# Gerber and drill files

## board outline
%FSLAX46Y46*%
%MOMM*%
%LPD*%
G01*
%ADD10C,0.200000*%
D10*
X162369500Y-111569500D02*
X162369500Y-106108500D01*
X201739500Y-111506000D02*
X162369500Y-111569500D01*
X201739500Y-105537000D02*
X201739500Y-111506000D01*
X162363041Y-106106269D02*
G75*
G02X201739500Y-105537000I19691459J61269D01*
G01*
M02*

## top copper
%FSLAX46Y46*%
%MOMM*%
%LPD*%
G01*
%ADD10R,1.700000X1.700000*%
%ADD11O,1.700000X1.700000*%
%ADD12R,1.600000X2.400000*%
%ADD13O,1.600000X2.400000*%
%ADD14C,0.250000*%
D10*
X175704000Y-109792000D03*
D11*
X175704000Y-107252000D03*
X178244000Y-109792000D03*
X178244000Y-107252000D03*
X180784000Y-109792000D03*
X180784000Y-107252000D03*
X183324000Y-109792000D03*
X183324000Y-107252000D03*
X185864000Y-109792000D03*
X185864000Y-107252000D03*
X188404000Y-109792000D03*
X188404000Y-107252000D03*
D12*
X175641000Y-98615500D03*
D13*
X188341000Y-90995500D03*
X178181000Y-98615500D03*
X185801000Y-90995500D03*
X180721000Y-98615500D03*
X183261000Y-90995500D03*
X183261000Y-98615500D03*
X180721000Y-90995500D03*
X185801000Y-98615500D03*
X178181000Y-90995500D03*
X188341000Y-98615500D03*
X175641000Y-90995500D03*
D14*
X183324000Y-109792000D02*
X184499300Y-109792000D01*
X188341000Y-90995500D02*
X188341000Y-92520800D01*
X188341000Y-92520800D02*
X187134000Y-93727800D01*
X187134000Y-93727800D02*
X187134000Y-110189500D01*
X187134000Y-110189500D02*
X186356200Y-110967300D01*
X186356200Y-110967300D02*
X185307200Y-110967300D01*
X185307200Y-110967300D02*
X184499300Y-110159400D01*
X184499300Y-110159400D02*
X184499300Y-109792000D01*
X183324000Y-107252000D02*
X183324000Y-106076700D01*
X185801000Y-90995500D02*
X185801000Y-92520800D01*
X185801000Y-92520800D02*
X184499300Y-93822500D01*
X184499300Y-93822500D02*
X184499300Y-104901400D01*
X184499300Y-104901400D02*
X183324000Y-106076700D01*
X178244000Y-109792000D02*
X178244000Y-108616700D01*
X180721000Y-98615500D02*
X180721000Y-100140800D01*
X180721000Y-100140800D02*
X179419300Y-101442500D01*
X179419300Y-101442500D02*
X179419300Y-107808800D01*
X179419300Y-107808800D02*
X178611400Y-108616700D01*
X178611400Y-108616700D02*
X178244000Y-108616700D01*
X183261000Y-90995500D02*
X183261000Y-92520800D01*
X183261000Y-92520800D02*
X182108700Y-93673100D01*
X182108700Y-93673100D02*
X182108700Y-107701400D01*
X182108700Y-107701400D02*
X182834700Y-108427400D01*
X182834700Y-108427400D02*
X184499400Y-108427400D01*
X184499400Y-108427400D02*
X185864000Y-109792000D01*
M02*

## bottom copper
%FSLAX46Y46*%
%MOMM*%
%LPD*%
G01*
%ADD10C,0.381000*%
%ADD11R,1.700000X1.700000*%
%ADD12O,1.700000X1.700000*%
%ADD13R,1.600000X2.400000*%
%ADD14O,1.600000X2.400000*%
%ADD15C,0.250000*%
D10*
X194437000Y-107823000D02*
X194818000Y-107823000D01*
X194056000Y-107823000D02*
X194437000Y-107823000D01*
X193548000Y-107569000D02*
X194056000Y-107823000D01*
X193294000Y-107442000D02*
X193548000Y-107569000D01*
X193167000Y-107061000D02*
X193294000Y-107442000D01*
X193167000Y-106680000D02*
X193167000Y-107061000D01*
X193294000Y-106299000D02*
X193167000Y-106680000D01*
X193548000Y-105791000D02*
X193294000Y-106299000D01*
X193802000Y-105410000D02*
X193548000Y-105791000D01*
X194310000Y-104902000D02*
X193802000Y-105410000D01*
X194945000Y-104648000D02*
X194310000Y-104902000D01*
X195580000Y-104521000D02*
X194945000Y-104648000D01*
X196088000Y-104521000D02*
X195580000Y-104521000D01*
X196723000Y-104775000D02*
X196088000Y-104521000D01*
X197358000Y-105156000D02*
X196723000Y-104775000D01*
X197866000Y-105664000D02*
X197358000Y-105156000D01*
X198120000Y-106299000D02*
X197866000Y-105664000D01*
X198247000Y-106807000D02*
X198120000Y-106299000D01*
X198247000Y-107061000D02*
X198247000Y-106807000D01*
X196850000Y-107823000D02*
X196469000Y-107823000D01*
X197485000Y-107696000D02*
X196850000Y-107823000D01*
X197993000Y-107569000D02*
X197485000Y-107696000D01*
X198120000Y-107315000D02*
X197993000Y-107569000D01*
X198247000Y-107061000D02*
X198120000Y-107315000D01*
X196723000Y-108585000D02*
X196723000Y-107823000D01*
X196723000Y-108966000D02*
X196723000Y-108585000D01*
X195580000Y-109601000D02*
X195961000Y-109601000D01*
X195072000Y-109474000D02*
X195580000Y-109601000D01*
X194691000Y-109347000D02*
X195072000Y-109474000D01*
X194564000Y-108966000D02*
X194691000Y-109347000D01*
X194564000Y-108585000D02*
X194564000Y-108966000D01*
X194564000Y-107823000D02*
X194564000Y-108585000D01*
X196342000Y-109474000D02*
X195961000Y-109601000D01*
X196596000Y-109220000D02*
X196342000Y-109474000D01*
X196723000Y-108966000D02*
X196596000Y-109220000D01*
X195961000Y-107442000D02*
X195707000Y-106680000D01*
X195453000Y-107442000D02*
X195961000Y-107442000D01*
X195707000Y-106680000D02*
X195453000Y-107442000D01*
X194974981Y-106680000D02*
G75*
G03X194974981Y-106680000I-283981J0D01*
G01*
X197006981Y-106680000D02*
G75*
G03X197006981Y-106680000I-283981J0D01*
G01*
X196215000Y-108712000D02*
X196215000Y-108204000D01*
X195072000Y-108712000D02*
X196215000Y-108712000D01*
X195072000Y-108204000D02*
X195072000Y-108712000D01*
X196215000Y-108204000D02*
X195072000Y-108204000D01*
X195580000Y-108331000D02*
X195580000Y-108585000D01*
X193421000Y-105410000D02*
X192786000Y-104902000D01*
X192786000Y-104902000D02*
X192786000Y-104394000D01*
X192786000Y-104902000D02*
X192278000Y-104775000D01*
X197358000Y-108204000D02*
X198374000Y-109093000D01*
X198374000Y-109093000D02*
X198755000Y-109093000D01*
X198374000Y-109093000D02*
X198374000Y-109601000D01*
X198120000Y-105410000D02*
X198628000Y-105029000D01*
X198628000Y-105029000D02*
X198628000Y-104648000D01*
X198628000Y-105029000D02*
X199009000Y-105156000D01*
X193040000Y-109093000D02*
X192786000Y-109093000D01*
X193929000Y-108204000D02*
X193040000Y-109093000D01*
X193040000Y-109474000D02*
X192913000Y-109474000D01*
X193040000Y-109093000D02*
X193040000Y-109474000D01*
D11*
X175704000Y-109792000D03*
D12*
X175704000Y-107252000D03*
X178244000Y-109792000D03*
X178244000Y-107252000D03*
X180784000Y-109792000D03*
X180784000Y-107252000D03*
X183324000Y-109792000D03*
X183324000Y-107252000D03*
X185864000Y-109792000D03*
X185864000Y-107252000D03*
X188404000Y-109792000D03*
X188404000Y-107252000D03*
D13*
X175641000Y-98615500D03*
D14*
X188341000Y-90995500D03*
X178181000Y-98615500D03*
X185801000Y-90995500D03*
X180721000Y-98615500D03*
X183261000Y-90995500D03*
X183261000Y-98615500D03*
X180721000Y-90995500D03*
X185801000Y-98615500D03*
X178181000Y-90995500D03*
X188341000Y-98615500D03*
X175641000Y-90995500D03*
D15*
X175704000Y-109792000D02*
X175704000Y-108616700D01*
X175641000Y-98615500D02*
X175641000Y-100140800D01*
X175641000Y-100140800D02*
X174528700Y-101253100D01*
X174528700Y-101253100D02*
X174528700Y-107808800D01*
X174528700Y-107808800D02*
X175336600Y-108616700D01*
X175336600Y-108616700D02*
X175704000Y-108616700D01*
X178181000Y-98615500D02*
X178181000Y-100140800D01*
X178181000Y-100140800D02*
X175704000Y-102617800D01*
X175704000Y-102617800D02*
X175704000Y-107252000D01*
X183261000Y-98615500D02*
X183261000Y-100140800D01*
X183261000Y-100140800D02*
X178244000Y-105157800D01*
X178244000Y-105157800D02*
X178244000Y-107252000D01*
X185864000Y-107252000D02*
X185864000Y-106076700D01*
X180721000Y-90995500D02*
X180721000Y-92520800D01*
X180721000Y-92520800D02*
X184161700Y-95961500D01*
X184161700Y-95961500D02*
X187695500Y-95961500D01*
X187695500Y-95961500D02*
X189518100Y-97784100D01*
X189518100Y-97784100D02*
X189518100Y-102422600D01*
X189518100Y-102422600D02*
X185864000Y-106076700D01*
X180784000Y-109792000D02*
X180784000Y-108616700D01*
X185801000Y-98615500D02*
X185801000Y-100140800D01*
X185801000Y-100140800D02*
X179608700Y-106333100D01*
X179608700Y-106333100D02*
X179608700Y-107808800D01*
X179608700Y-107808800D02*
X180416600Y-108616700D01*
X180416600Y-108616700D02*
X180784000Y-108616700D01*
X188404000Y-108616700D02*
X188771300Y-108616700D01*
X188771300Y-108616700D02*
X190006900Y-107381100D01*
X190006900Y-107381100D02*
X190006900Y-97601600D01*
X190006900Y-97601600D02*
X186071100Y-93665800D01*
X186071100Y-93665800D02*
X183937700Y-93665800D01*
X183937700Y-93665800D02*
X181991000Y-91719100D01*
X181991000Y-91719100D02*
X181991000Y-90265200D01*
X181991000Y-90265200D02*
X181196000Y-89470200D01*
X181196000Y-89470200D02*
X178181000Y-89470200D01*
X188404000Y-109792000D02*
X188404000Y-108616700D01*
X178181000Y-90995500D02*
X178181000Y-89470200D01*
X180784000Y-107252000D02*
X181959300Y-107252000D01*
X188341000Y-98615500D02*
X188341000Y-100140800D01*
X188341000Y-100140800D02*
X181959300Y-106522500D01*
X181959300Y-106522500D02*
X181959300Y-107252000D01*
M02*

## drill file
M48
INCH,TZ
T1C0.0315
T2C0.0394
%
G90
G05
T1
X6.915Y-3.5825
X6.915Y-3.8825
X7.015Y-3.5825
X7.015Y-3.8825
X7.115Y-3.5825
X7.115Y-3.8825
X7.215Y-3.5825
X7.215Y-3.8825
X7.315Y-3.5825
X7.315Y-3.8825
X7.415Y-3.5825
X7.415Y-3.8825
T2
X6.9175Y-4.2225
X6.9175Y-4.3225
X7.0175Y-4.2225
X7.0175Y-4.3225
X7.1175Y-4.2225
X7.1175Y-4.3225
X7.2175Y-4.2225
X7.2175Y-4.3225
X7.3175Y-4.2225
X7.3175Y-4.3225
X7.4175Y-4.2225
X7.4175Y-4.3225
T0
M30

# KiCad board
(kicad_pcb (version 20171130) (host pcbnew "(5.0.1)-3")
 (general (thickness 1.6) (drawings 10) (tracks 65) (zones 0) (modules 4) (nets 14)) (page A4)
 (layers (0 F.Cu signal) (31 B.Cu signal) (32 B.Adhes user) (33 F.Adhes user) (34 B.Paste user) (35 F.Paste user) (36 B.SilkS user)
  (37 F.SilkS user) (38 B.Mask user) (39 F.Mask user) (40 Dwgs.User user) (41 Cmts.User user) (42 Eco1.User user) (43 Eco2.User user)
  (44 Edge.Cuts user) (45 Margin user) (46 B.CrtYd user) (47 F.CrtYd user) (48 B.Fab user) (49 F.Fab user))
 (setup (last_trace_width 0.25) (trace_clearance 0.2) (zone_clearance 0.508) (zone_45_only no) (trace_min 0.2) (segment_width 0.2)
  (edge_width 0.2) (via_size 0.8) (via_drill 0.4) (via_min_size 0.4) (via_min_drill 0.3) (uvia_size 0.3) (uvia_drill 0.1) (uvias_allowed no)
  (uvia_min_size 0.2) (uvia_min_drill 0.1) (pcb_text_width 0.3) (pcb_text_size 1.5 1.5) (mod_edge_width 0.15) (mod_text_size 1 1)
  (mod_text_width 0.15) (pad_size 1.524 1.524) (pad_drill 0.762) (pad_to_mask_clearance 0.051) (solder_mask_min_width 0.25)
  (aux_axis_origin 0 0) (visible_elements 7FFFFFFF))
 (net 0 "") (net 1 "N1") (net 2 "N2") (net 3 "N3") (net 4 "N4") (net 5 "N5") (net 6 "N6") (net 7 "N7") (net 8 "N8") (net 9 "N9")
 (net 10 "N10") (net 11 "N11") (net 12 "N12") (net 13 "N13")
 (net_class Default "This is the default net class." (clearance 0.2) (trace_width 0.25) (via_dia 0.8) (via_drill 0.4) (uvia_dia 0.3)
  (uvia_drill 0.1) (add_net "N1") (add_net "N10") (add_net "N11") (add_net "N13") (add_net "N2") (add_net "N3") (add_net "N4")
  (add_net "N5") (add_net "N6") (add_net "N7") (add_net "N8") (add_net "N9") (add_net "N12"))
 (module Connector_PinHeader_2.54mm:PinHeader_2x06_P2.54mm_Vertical (layer F.Cu) (at 175.704 109.792 90)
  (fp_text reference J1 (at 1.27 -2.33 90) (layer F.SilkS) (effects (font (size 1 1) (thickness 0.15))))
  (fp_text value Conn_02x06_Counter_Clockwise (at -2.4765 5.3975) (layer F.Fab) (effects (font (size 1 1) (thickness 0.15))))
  (pad 1 thru_hole rect (at 0 0 90) (size 1.7 1.7) (drill 1) (layers *.Cu *.Mask) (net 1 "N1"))
  (pad 2 thru_hole oval (at 2.54 0 90) (size 1.7 1.7) (drill 1) (layers *.Cu *.Mask) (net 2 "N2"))
  (pad 3 thru_hole oval (at 0 2.54 90) (size 1.7 1.7) (drill 1) (layers *.Cu *.Mask) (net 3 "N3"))
  (pad 4 thru_hole oval (at 2.54 2.54 90) (size 1.7 1.7) (drill 1) (layers *.Cu *.Mask) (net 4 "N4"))
  (pad 5 thru_hole oval (at 0 5.08 90) (size 1.7 1.7) (drill 1) (layers *.Cu *.Mask) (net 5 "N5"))
  (pad 6 thru_hole oval (at 2.54 5.08 90) (size 1.7 1.7) (drill 1) (layers *.Cu *.Mask) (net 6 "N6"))
  (pad 7 thru_hole oval (at 0 7.62 90) (size 1.7 1.7) (drill 1) (layers *.Cu *.Mask) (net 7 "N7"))
  (pad 8 thru_hole oval (at 2.54 7.62 90) (size 1.7 1.7) (drill 1) (layers *.Cu *.Mask) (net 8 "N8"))
  (pad 9 thru_hole oval (at 0 10.16 90) (size 1.7 1.7) (drill 1) (layers *.Cu *.Mask) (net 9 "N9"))
  (pad 10 thru_hole oval (at 2.54 10.16 90) (size 1.7 1.7) (drill 1) (layers *.Cu *.Mask) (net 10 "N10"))
  (pad 11 thru_hole oval (at 0 12.7 90) (size 1.7 1.7) (drill 1) (layers *.Cu *.Mask) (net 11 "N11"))
  (pad 12 thru_hole oval (at 2.54 12.7 90) (size 1.7 1.7) (drill 1) (layers *.Cu *.Mask) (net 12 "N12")))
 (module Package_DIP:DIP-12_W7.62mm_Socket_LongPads (layer F.Cu) (at 175.641 98.6155 90)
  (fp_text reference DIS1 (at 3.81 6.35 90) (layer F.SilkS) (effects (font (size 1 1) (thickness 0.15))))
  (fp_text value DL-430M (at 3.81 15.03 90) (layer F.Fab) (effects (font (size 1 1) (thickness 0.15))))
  (pad 1 thru_hole rect (at 0 0 90) (size 2.4 1.6) (drill 0.8) (layers *.Cu *.Mask) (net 1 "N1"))
  (pad 7 thru_hole oval (at 7.62 12.7 90) (size 2.4 1.6) (drill 0.8) (layers *.Cu *.Mask) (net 7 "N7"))
  (pad 2 thru_hole oval (at 0 2.54 90) (size 2.4 1.6) (drill 0.8) (layers *.Cu *.Mask) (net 2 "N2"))
  (pad 8 thru_hole oval (at 7.62 10.16 90) (size 2.4 1.6) (drill 0.8) (layers *.Cu *.Mask) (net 8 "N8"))
  (pad 3 thru_hole oval (at 0 5.08 90) (size 2.4 1.6) (drill 0.8) (layers *.Cu *.Mask) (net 3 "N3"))
  (pad 9 thru_hole oval (at 7.62 7.62 90) (size 2.4 1.6) (drill 0.8) (layers *.Cu *.Mask) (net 9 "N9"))
  (pad 4 thru_hole oval (at 0 7.62 90) (size 2.4 1.6) (drill 0.8) (layers *.Cu *.Mask) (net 4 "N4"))
  (pad 10 thru_hole oval (at 7.62 5.08 90) (size 2.4 1.6) (drill 0.8) (layers *.Cu *.Mask) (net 10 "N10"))
  (pad 5 thru_hole oval (at 0 10.16 90) (size 2.4 1.6) (drill 0.8) (layers *.Cu *.Mask) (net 5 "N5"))
  (pad 11 thru_hole oval (at 7.62 2.54 90) (size 2.4 1.6) (drill 0.8) (layers *.Cu *.Mask) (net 11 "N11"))
  (pad 6 thru_hole oval (at 0 12.7 90) (size 2.4 1.6) (drill 0.8) (layers *.Cu *.Mask) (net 6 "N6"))
  (pad 12 thru_hole oval (at 7.62 0 90) (size 2.4 1.6) (drill 0.8) (layers *.Cu *.Mask) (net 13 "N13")))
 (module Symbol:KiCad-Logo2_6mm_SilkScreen (layer B.Cu) (at 182.3085 102.8065 180)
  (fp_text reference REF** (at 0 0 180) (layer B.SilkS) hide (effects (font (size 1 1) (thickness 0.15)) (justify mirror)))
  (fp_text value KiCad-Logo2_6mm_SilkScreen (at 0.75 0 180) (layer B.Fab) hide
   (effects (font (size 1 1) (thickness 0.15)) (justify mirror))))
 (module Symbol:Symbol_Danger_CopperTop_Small (layer B.Cu) (at 195.707 107.061 180)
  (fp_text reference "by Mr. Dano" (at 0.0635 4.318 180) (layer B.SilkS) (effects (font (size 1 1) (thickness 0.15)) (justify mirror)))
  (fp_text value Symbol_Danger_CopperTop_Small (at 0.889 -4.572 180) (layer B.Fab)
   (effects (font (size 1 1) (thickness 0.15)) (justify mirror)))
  (fp_line (start 1.27 -0.762) (end 0.889 -0.762) (layer B.Cu) (width 0.381))
  (fp_line (start 1.651 -0.762) (end 1.27 -0.762) (layer B.Cu) (width 0.381))
  (fp_line (start 2.159 -0.508) (end 1.651 -0.762) (layer B.Cu) (width 0.381))
  (fp_line (start 2.413 -0.381) (end 2.159 -0.508) (layer B.Cu) (width 0.381))
  (fp_line (start 2.54 0) (end 2.413 -0.381) (layer B.Cu) (width 0.381))
  (fp_line (start 2.54 0.381) (end 2.54 0) (layer B.Cu) (width 0.381))
  (fp_line (start 2.413 0.762) (end 2.54 0.381) (layer B.Cu) (width 0.381))
  (fp_line (start 2.159 1.27) (end 2.413 0.762) (layer B.Cu) (width 0.381))
  (fp_line (start 1.905 1.651) (end 2.159 1.27) (layer B.Cu) (width 0.381))
  (fp_line (start 1.397 2.159) (end 1.905 1.651) (layer B.Cu) (width 0.381))
  (fp_line (start 0.762 2.413) (end 1.397 2.159) (layer B.Cu) (width 0.381))
  (fp_line (start 0.127 2.54) (end 0.762 2.413) (layer B.Cu) (width 0.381))
  (fp_line (start -0.381 2.54) (end 0.127 2.54) (layer B.Cu) (width 0.381))
  (fp_line (start -1.016 2.286) (end -0.381 2.54) (layer B.Cu) (width 0.381))
  (fp_line (start -1.651 1.905) (end -1.016 2.286) (layer B.Cu) (width 0.381))
  (fp_line (start -2.159 1.397) (end -1.651 1.905) (layer B.Cu) (width 0.381))
  (fp_line (start -2.413 0.762) (end -2.159 1.397) (layer B.Cu) (width 0.381))
  (fp_line (start -2.54 0.254) (end -2.413 0.762) (layer B.Cu) (width 0.381))
  (fp_line (start -2.54 0) (end -2.54 0.254) (layer B.Cu) (width 0.381))
  (fp_line (start -1.143 -0.762) (end -0.762 -0.762) (layer B.Cu) (width 0.381))
  (fp_line (start -1.778 -0.635) (end -1.143 -0.762) (layer B.Cu) (width 0.381))
  (fp_line (start -2.286 -0.508) (end -1.778 -0.635) (layer B.Cu) (width 0.381))
  (fp_line (start -2.413 -0.254) (end -2.286 -0.508) (layer B.Cu) (width 0.381))
  (fp_line (start -2.54 0) (end -2.413 -0.254) (layer B.Cu) (width 0.381))
  (fp_line (start -1.016 -1.524) (end -1.016 -0.762) (layer B.Cu) (width 0.381))
  (fp_line (start -1.016 -1.905) (end -1.016 -1.524) (layer B.Cu) (width 0.381))
  (fp_line (start 0.127 -2.54) (end -0.254 -2.54) (layer B.Cu) (width 0.381))
  (fp_line (start 0.635 -2.413) (end 0.127 -2.54) (layer B.Cu) (width 0.381))
  (fp_line (start 1.016 -2.286) (end 0.635 -2.413) (layer B.Cu) (width 0.381))
  (fp_line (start 1.143 -1.905) (end 1.016 -2.286) (layer B.Cu) (width 0.381))
  (fp_line (start 1.143 -1.524) (end 1.143 -1.905) (layer B.Cu) (width 0.381))
  (fp_line (start 1.143 -0.762) (end 1.143 -1.524) (layer B.Cu) (width 0.381))
  (fp_line (start -0.635 -2.413) (end -0.254 -2.54) (layer B.Cu) (width 0.381))
  (fp_line (start -0.889 -2.159) (end -0.635 -2.413) (layer B.Cu) (width 0.381))
  (fp_line (start -1.016 -1.905) (end -0.889 -2.159) (layer B.Cu) (width 0.381))
  (fp_line (start -0.254 -0.381) (end 0 0.381) (layer B.Cu) (width 0.381))
  (fp_line (start 0.254 -0.381) (end -0.254 -0.381) (layer B.Cu) (width 0.381))
  (fp_line (start 0 0.381) (end 0.254 -0.381) (layer B.Cu) (width 0.381))
  (fp_circle (center 1.016 0.381) (end 1.27 0.254) (layer B.Cu) (width 0.381))
  (fp_circle (center -1.016 0.381) (end -1.27 0.254) (layer B.Cu) (width 0.381))
  (fp_line (start -0.508 -1.651) (end -0.508 -1.143) (layer B.Cu) (width 0.381))
  (fp_line (start 0.635 -1.651) (end -0.508 -1.651) (layer B.Cu) (width 0.381))
  (fp_line (start 0.635 -1.143) (end 0.635 -1.651) (layer B.Cu) (width 0.381))
  (fp_line (start -0.508 -1.143) (end 0.635 -1.143) (layer B.Cu) (width 0.381))
  (fp_line (start 0.127 -1.27) (end 0.127 -1.524) (layer B.Cu) (width 0.381))
  (fp_line (start 2.286 1.651) (end 2.921 2.159) (layer B.Cu) (width 0.381))
  (fp_line (start 2.921 2.159) (end 2.921 2.667) (layer B.Cu) (width 0.381))
  (fp_line (start 2.921 2.159) (end 3.429 2.286) (layer B.Cu) (width 0.381))
  (fp_line (start -1.651 -1.143) (end -2.667 -2.032) (layer B.Cu) (width 0.381))
  (fp_line (start -2.667 -2.032) (end -3.048 -2.032) (layer B.Cu) (width 0.381))
  (fp_line (start -2.667 -2.032) (end -2.667 -2.54) (layer B.Cu) (width 0.381))
  (fp_line (start -2.413 1.651) (end -2.921 2.032) (layer B.Cu) (width 0.381))
  (fp_line (start -2.921 2.032) (end -2.921 2.413) (layer B.Cu) (width 0.381))
  (fp_line (start -2.921 2.032) (end -3.302 1.905) (layer B.Cu) (width 0.381))
  (fp_line (start 2.667 -2.032) (end 2.921 -2.032) (layer B.Cu) (width 0.381))
  (fp_line (start 1.778 -1.143) (end 2.667 -2.032) (layer B.Cu) (width 0.381))
  (fp_line (start 2.667 -2.413) (end 2.794 -2.413) (layer B.Cu) (width 0.381))
  (fp_line (start 2.667 -2.032) (end 2.667 -2.413) (layer B.Cu) (width 0.381)))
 (gr_line (start 162.3695 111.5695) (end 162.3695 106.1085) (layer Edge.Cuts) (width 0.2))
 (gr_line (start 201.7395 111.506) (end 162.3695 111.5695) (layer Edge.Cuts) (width 0.2))
 (gr_line (start 201.7395 105.537) (end 201.7395 111.506) (layer Edge.Cuts) (width 0.2))
 (gr_arc (start 182.0545 106.045) (end 201.7395 105.537) (angle -178.7) (layer Edge.Cuts) (width 0.2))
 (segment (start 175.704 109.792) (end 175.704 108.6167) (width 0.25) (layer B.Cu) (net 1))
 (segment (start 175.641 98.6155) (end 175.641 100.1408) (width 0.25) (layer B.Cu) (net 1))
 (segment (start 175.641 100.1408) (end 174.5287 101.2531) (width 0.25) (layer B.Cu) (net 1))
 (segment (start 174.5287 101.2531) (end 174.5287 107.8088) (width 0.25) (layer B.Cu) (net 1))
 (segment (start 174.5287 107.8088) (end 175.3366 108.6167) (width 0.25) (layer B.Cu) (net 1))
 (segment (start 175.3366 108.6167) (end 175.704 108.6167) (width 0.25) (layer B.Cu) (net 1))
 (segment (start 183.324 109.792) (end 184.4993 109.792) (width 0.25) (layer F.Cu) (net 7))
 (segment (start 188.341 90.9955) (end 188.341 92.5208) (width 0.25) (layer F.Cu) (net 7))
 (segment (start 188.341 92.5208) (end 187.134 93.7278) (width 0.25) (layer F.Cu) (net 7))
 (segment (start 187.134 93.7278) (end 187.134 110.1895) (width 0.25) (layer F.Cu) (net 7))
 (segment (start 187.134 110.1895) (end 186.3562 110.9673) (width 0.25) (layer F.Cu) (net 7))
 (segment (start 186.3562 110.9673) (end 185.3072 110.9673) (width 0.25) (layer F.Cu) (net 7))
 (segment (start 185.3072 110.9673) (end 184.4993 110.1594) (width 0.25) (layer F.Cu) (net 7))
 (segment (start 184.4993 110.1594) (end 184.4993 109.792) (width 0.25) (layer F.Cu) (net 7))
 (segment (start 178.181 98.6155) (end 178.181 100.1408) (width 0.25) (layer B.Cu) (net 2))
 (segment (start 178.181 100.1408) (end 175.704 102.6178) (width 0.25) (layer B.Cu) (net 2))
 (segment (start 175.704 102.6178) (end 175.704 107.252) (width 0.25) (layer B.Cu) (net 2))
 (segment (start 183.324 107.252) (end 183.324 106.0767) (width 0.25) (layer F.Cu) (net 8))
 (segment (start 185.801 90.9955) (end 185.801 92.5208) (width 0.25) (layer F.Cu) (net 8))
 (segment (start 185.801 92.5208) (end 184.4993 93.8225) (width 0.25) (layer F.Cu) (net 8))
 (segment (start 184.4993 93.8225) (end 184.4993 104.9014) (width 0.25) (layer F.Cu) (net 8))
 (segment (start 184.4993 104.9014) (end 183.324 106.0767) (width 0.25) (layer F.Cu) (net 8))
 (segment (start 178.244 109.792) (end 178.244 108.6167) (width 0.25) (layer F.Cu) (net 3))
 (segment (start 180.721 98.6155) (end 180.721 100.1408) (width 0.25) (layer F.Cu) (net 3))
 (segment (start 180.721 100.1408) (end 179.4193 101.4425) (width 0.25) (layer F.Cu) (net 3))
 (segment (start 179.4193 101.4425) (end 179.4193 107.8088) (width 0.25) (layer F.Cu) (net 3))
 (segment (start 179.4193 107.8088) (end 178.6114 108.6167) (width 0.25) (layer F.Cu) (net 3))
 (segment (start 178.6114 108.6167) (end 178.244 108.6167) (width 0.25) (layer F.Cu) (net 3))
 (segment (start 183.261 90.9955) (end 183.261 92.5208) (width 0.25) (layer F.Cu) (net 9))
 (segment (start 183.261 92.5208) (end 182.1087 93.6731) (width 0.25) (layer F.Cu) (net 9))
 (segment (start 182.1087 93.6731) (end 182.1087 107.7014) (width 0.25) (layer F.Cu) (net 9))
 (segment (start 182.1087 107.7014) (end 182.8347 108.4274) (width 0.25) (layer F.Cu) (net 9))
 (segment (start 182.8347 108.4274) (end 184.4994 108.4274) (width 0.25) (layer F.Cu) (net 9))
 (segment (start 184.4994 108.4274) (end 185.864 109.792) (width 0.25) (layer F.Cu) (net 9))
 (segment (start 183.261 98.6155) (end 183.261 100.1408) (width 0.25) (layer B.Cu) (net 4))
 (segment (start 183.261 100.1408) (end 178.244 105.1578) (width 0.25) (layer B.Cu) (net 4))
 (segment (start 178.244 105.1578) (end 178.244 107.252) (width 0.25) (layer B.Cu) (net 4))
 (segment (start 185.864 107.252) (end 185.864 106.0767) (width 0.25) (layer B.Cu) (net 10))
 (segment (start 180.721 90.9955) (end 180.721 92.5208) (width 0.25) (layer B.Cu) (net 10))
 (segment (start 180.721 92.5208) (end 184.1617 95.9615) (width 0.25) (layer B.Cu) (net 10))
 (segment (start 184.1617 95.9615) (end 187.6955 95.9615) (width 0.25) (layer B.Cu) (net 10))
 (segment (start 187.6955 95.9615) (end 189.5181 97.7841) (width 0.25) (layer B.Cu) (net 10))
 (segment (start 189.5181 97.7841) (end 189.5181 102.4226) (width 0.25) (layer B.Cu) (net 10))
 (segment (start 189.5181 102.4226) (end 185.864 106.0767) (width 0.25) (layer B.Cu) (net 10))
 (segment (start 180.784 109.792) (end 180.784 108.6167) (width 0.25) (layer B.Cu) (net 5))
 (segment (start 185.801 98.6155) (end 185.801 100.1408) (width 0.25) (layer B.Cu) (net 5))
 (segment (start 185.801 100.1408) (end 179.6087 106.3331) (width 0.25) (layer B.Cu) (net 5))
 (segment (start 179.6087 106.3331) (end 179.6087 107.8088) (width 0.25) (layer B.Cu) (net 5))
 (segment (start 179.6087 107.8088) (end 180.4166 108.6167) (width 0.25) (layer B.Cu) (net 5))
 (segment (start 180.4166 108.6167) (end 180.784 108.6167) (width 0.25) (layer B.Cu) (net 5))
 (segment (start 188.404 108.6167) (end 188.7713 108.6167) (width 0.25) (layer B.Cu) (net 11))
 (segment (start 188.7713 108.6167) (end 190.0069 107.3811) (width 0.25) (layer B.Cu) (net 11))
 (segment (start 190.0069 107.3811) (end 190.0069 97.6016) (width 0.25) (layer B.Cu) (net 11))
 (segment (start 190.0069 97.6016) (end 186.0711 93.6658) (width 0.25) (layer B.Cu) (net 11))
 (segment (start 186.0711 93.6658) (end 183.9377 93.6658) (width 0.25) (layer B.Cu) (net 11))
 (segment (start 183.9377 93.6658) (end 181.991 91.7191) (width 0.25) (layer B.Cu) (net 11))
 (segment (start 181.991 91.7191) (end 181.991 90.2652) (width 0.25) (layer B.Cu) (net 11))
 (segment (start 181.991 90.2652) (end 181.196 89.4702) (width 0.25) (layer B.Cu) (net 11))
 (segment (start 181.196 89.4702) (end 178.181 89.4702) (width 0.25) (layer B.Cu) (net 11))
 (segment (start 188.404 109.792) (end 188.404 108.6167) (width 0.25) (layer B.Cu) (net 11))
 (segment (start 178.181 90.9955) (end 178.181 89.4702) (width 0.25) (layer B.Cu) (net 11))
 (segment (start 180.784 107.252) (end 181.9593 107.252) (width 0.25) (layer B.Cu) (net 6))
 (segment (start 188.341 98.6155) (end 188.341 100.1408) (width 0.25) (layer B.Cu) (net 6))
 (segment (start 188.341 100.1408) (end 181.9593 106.5225) (width 0.25) (layer B.Cu) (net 6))
 (segment (start 181.9593 106.5225) (end 181.9593 107.252) (width 0.25) (layer B.Cu) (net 6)))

